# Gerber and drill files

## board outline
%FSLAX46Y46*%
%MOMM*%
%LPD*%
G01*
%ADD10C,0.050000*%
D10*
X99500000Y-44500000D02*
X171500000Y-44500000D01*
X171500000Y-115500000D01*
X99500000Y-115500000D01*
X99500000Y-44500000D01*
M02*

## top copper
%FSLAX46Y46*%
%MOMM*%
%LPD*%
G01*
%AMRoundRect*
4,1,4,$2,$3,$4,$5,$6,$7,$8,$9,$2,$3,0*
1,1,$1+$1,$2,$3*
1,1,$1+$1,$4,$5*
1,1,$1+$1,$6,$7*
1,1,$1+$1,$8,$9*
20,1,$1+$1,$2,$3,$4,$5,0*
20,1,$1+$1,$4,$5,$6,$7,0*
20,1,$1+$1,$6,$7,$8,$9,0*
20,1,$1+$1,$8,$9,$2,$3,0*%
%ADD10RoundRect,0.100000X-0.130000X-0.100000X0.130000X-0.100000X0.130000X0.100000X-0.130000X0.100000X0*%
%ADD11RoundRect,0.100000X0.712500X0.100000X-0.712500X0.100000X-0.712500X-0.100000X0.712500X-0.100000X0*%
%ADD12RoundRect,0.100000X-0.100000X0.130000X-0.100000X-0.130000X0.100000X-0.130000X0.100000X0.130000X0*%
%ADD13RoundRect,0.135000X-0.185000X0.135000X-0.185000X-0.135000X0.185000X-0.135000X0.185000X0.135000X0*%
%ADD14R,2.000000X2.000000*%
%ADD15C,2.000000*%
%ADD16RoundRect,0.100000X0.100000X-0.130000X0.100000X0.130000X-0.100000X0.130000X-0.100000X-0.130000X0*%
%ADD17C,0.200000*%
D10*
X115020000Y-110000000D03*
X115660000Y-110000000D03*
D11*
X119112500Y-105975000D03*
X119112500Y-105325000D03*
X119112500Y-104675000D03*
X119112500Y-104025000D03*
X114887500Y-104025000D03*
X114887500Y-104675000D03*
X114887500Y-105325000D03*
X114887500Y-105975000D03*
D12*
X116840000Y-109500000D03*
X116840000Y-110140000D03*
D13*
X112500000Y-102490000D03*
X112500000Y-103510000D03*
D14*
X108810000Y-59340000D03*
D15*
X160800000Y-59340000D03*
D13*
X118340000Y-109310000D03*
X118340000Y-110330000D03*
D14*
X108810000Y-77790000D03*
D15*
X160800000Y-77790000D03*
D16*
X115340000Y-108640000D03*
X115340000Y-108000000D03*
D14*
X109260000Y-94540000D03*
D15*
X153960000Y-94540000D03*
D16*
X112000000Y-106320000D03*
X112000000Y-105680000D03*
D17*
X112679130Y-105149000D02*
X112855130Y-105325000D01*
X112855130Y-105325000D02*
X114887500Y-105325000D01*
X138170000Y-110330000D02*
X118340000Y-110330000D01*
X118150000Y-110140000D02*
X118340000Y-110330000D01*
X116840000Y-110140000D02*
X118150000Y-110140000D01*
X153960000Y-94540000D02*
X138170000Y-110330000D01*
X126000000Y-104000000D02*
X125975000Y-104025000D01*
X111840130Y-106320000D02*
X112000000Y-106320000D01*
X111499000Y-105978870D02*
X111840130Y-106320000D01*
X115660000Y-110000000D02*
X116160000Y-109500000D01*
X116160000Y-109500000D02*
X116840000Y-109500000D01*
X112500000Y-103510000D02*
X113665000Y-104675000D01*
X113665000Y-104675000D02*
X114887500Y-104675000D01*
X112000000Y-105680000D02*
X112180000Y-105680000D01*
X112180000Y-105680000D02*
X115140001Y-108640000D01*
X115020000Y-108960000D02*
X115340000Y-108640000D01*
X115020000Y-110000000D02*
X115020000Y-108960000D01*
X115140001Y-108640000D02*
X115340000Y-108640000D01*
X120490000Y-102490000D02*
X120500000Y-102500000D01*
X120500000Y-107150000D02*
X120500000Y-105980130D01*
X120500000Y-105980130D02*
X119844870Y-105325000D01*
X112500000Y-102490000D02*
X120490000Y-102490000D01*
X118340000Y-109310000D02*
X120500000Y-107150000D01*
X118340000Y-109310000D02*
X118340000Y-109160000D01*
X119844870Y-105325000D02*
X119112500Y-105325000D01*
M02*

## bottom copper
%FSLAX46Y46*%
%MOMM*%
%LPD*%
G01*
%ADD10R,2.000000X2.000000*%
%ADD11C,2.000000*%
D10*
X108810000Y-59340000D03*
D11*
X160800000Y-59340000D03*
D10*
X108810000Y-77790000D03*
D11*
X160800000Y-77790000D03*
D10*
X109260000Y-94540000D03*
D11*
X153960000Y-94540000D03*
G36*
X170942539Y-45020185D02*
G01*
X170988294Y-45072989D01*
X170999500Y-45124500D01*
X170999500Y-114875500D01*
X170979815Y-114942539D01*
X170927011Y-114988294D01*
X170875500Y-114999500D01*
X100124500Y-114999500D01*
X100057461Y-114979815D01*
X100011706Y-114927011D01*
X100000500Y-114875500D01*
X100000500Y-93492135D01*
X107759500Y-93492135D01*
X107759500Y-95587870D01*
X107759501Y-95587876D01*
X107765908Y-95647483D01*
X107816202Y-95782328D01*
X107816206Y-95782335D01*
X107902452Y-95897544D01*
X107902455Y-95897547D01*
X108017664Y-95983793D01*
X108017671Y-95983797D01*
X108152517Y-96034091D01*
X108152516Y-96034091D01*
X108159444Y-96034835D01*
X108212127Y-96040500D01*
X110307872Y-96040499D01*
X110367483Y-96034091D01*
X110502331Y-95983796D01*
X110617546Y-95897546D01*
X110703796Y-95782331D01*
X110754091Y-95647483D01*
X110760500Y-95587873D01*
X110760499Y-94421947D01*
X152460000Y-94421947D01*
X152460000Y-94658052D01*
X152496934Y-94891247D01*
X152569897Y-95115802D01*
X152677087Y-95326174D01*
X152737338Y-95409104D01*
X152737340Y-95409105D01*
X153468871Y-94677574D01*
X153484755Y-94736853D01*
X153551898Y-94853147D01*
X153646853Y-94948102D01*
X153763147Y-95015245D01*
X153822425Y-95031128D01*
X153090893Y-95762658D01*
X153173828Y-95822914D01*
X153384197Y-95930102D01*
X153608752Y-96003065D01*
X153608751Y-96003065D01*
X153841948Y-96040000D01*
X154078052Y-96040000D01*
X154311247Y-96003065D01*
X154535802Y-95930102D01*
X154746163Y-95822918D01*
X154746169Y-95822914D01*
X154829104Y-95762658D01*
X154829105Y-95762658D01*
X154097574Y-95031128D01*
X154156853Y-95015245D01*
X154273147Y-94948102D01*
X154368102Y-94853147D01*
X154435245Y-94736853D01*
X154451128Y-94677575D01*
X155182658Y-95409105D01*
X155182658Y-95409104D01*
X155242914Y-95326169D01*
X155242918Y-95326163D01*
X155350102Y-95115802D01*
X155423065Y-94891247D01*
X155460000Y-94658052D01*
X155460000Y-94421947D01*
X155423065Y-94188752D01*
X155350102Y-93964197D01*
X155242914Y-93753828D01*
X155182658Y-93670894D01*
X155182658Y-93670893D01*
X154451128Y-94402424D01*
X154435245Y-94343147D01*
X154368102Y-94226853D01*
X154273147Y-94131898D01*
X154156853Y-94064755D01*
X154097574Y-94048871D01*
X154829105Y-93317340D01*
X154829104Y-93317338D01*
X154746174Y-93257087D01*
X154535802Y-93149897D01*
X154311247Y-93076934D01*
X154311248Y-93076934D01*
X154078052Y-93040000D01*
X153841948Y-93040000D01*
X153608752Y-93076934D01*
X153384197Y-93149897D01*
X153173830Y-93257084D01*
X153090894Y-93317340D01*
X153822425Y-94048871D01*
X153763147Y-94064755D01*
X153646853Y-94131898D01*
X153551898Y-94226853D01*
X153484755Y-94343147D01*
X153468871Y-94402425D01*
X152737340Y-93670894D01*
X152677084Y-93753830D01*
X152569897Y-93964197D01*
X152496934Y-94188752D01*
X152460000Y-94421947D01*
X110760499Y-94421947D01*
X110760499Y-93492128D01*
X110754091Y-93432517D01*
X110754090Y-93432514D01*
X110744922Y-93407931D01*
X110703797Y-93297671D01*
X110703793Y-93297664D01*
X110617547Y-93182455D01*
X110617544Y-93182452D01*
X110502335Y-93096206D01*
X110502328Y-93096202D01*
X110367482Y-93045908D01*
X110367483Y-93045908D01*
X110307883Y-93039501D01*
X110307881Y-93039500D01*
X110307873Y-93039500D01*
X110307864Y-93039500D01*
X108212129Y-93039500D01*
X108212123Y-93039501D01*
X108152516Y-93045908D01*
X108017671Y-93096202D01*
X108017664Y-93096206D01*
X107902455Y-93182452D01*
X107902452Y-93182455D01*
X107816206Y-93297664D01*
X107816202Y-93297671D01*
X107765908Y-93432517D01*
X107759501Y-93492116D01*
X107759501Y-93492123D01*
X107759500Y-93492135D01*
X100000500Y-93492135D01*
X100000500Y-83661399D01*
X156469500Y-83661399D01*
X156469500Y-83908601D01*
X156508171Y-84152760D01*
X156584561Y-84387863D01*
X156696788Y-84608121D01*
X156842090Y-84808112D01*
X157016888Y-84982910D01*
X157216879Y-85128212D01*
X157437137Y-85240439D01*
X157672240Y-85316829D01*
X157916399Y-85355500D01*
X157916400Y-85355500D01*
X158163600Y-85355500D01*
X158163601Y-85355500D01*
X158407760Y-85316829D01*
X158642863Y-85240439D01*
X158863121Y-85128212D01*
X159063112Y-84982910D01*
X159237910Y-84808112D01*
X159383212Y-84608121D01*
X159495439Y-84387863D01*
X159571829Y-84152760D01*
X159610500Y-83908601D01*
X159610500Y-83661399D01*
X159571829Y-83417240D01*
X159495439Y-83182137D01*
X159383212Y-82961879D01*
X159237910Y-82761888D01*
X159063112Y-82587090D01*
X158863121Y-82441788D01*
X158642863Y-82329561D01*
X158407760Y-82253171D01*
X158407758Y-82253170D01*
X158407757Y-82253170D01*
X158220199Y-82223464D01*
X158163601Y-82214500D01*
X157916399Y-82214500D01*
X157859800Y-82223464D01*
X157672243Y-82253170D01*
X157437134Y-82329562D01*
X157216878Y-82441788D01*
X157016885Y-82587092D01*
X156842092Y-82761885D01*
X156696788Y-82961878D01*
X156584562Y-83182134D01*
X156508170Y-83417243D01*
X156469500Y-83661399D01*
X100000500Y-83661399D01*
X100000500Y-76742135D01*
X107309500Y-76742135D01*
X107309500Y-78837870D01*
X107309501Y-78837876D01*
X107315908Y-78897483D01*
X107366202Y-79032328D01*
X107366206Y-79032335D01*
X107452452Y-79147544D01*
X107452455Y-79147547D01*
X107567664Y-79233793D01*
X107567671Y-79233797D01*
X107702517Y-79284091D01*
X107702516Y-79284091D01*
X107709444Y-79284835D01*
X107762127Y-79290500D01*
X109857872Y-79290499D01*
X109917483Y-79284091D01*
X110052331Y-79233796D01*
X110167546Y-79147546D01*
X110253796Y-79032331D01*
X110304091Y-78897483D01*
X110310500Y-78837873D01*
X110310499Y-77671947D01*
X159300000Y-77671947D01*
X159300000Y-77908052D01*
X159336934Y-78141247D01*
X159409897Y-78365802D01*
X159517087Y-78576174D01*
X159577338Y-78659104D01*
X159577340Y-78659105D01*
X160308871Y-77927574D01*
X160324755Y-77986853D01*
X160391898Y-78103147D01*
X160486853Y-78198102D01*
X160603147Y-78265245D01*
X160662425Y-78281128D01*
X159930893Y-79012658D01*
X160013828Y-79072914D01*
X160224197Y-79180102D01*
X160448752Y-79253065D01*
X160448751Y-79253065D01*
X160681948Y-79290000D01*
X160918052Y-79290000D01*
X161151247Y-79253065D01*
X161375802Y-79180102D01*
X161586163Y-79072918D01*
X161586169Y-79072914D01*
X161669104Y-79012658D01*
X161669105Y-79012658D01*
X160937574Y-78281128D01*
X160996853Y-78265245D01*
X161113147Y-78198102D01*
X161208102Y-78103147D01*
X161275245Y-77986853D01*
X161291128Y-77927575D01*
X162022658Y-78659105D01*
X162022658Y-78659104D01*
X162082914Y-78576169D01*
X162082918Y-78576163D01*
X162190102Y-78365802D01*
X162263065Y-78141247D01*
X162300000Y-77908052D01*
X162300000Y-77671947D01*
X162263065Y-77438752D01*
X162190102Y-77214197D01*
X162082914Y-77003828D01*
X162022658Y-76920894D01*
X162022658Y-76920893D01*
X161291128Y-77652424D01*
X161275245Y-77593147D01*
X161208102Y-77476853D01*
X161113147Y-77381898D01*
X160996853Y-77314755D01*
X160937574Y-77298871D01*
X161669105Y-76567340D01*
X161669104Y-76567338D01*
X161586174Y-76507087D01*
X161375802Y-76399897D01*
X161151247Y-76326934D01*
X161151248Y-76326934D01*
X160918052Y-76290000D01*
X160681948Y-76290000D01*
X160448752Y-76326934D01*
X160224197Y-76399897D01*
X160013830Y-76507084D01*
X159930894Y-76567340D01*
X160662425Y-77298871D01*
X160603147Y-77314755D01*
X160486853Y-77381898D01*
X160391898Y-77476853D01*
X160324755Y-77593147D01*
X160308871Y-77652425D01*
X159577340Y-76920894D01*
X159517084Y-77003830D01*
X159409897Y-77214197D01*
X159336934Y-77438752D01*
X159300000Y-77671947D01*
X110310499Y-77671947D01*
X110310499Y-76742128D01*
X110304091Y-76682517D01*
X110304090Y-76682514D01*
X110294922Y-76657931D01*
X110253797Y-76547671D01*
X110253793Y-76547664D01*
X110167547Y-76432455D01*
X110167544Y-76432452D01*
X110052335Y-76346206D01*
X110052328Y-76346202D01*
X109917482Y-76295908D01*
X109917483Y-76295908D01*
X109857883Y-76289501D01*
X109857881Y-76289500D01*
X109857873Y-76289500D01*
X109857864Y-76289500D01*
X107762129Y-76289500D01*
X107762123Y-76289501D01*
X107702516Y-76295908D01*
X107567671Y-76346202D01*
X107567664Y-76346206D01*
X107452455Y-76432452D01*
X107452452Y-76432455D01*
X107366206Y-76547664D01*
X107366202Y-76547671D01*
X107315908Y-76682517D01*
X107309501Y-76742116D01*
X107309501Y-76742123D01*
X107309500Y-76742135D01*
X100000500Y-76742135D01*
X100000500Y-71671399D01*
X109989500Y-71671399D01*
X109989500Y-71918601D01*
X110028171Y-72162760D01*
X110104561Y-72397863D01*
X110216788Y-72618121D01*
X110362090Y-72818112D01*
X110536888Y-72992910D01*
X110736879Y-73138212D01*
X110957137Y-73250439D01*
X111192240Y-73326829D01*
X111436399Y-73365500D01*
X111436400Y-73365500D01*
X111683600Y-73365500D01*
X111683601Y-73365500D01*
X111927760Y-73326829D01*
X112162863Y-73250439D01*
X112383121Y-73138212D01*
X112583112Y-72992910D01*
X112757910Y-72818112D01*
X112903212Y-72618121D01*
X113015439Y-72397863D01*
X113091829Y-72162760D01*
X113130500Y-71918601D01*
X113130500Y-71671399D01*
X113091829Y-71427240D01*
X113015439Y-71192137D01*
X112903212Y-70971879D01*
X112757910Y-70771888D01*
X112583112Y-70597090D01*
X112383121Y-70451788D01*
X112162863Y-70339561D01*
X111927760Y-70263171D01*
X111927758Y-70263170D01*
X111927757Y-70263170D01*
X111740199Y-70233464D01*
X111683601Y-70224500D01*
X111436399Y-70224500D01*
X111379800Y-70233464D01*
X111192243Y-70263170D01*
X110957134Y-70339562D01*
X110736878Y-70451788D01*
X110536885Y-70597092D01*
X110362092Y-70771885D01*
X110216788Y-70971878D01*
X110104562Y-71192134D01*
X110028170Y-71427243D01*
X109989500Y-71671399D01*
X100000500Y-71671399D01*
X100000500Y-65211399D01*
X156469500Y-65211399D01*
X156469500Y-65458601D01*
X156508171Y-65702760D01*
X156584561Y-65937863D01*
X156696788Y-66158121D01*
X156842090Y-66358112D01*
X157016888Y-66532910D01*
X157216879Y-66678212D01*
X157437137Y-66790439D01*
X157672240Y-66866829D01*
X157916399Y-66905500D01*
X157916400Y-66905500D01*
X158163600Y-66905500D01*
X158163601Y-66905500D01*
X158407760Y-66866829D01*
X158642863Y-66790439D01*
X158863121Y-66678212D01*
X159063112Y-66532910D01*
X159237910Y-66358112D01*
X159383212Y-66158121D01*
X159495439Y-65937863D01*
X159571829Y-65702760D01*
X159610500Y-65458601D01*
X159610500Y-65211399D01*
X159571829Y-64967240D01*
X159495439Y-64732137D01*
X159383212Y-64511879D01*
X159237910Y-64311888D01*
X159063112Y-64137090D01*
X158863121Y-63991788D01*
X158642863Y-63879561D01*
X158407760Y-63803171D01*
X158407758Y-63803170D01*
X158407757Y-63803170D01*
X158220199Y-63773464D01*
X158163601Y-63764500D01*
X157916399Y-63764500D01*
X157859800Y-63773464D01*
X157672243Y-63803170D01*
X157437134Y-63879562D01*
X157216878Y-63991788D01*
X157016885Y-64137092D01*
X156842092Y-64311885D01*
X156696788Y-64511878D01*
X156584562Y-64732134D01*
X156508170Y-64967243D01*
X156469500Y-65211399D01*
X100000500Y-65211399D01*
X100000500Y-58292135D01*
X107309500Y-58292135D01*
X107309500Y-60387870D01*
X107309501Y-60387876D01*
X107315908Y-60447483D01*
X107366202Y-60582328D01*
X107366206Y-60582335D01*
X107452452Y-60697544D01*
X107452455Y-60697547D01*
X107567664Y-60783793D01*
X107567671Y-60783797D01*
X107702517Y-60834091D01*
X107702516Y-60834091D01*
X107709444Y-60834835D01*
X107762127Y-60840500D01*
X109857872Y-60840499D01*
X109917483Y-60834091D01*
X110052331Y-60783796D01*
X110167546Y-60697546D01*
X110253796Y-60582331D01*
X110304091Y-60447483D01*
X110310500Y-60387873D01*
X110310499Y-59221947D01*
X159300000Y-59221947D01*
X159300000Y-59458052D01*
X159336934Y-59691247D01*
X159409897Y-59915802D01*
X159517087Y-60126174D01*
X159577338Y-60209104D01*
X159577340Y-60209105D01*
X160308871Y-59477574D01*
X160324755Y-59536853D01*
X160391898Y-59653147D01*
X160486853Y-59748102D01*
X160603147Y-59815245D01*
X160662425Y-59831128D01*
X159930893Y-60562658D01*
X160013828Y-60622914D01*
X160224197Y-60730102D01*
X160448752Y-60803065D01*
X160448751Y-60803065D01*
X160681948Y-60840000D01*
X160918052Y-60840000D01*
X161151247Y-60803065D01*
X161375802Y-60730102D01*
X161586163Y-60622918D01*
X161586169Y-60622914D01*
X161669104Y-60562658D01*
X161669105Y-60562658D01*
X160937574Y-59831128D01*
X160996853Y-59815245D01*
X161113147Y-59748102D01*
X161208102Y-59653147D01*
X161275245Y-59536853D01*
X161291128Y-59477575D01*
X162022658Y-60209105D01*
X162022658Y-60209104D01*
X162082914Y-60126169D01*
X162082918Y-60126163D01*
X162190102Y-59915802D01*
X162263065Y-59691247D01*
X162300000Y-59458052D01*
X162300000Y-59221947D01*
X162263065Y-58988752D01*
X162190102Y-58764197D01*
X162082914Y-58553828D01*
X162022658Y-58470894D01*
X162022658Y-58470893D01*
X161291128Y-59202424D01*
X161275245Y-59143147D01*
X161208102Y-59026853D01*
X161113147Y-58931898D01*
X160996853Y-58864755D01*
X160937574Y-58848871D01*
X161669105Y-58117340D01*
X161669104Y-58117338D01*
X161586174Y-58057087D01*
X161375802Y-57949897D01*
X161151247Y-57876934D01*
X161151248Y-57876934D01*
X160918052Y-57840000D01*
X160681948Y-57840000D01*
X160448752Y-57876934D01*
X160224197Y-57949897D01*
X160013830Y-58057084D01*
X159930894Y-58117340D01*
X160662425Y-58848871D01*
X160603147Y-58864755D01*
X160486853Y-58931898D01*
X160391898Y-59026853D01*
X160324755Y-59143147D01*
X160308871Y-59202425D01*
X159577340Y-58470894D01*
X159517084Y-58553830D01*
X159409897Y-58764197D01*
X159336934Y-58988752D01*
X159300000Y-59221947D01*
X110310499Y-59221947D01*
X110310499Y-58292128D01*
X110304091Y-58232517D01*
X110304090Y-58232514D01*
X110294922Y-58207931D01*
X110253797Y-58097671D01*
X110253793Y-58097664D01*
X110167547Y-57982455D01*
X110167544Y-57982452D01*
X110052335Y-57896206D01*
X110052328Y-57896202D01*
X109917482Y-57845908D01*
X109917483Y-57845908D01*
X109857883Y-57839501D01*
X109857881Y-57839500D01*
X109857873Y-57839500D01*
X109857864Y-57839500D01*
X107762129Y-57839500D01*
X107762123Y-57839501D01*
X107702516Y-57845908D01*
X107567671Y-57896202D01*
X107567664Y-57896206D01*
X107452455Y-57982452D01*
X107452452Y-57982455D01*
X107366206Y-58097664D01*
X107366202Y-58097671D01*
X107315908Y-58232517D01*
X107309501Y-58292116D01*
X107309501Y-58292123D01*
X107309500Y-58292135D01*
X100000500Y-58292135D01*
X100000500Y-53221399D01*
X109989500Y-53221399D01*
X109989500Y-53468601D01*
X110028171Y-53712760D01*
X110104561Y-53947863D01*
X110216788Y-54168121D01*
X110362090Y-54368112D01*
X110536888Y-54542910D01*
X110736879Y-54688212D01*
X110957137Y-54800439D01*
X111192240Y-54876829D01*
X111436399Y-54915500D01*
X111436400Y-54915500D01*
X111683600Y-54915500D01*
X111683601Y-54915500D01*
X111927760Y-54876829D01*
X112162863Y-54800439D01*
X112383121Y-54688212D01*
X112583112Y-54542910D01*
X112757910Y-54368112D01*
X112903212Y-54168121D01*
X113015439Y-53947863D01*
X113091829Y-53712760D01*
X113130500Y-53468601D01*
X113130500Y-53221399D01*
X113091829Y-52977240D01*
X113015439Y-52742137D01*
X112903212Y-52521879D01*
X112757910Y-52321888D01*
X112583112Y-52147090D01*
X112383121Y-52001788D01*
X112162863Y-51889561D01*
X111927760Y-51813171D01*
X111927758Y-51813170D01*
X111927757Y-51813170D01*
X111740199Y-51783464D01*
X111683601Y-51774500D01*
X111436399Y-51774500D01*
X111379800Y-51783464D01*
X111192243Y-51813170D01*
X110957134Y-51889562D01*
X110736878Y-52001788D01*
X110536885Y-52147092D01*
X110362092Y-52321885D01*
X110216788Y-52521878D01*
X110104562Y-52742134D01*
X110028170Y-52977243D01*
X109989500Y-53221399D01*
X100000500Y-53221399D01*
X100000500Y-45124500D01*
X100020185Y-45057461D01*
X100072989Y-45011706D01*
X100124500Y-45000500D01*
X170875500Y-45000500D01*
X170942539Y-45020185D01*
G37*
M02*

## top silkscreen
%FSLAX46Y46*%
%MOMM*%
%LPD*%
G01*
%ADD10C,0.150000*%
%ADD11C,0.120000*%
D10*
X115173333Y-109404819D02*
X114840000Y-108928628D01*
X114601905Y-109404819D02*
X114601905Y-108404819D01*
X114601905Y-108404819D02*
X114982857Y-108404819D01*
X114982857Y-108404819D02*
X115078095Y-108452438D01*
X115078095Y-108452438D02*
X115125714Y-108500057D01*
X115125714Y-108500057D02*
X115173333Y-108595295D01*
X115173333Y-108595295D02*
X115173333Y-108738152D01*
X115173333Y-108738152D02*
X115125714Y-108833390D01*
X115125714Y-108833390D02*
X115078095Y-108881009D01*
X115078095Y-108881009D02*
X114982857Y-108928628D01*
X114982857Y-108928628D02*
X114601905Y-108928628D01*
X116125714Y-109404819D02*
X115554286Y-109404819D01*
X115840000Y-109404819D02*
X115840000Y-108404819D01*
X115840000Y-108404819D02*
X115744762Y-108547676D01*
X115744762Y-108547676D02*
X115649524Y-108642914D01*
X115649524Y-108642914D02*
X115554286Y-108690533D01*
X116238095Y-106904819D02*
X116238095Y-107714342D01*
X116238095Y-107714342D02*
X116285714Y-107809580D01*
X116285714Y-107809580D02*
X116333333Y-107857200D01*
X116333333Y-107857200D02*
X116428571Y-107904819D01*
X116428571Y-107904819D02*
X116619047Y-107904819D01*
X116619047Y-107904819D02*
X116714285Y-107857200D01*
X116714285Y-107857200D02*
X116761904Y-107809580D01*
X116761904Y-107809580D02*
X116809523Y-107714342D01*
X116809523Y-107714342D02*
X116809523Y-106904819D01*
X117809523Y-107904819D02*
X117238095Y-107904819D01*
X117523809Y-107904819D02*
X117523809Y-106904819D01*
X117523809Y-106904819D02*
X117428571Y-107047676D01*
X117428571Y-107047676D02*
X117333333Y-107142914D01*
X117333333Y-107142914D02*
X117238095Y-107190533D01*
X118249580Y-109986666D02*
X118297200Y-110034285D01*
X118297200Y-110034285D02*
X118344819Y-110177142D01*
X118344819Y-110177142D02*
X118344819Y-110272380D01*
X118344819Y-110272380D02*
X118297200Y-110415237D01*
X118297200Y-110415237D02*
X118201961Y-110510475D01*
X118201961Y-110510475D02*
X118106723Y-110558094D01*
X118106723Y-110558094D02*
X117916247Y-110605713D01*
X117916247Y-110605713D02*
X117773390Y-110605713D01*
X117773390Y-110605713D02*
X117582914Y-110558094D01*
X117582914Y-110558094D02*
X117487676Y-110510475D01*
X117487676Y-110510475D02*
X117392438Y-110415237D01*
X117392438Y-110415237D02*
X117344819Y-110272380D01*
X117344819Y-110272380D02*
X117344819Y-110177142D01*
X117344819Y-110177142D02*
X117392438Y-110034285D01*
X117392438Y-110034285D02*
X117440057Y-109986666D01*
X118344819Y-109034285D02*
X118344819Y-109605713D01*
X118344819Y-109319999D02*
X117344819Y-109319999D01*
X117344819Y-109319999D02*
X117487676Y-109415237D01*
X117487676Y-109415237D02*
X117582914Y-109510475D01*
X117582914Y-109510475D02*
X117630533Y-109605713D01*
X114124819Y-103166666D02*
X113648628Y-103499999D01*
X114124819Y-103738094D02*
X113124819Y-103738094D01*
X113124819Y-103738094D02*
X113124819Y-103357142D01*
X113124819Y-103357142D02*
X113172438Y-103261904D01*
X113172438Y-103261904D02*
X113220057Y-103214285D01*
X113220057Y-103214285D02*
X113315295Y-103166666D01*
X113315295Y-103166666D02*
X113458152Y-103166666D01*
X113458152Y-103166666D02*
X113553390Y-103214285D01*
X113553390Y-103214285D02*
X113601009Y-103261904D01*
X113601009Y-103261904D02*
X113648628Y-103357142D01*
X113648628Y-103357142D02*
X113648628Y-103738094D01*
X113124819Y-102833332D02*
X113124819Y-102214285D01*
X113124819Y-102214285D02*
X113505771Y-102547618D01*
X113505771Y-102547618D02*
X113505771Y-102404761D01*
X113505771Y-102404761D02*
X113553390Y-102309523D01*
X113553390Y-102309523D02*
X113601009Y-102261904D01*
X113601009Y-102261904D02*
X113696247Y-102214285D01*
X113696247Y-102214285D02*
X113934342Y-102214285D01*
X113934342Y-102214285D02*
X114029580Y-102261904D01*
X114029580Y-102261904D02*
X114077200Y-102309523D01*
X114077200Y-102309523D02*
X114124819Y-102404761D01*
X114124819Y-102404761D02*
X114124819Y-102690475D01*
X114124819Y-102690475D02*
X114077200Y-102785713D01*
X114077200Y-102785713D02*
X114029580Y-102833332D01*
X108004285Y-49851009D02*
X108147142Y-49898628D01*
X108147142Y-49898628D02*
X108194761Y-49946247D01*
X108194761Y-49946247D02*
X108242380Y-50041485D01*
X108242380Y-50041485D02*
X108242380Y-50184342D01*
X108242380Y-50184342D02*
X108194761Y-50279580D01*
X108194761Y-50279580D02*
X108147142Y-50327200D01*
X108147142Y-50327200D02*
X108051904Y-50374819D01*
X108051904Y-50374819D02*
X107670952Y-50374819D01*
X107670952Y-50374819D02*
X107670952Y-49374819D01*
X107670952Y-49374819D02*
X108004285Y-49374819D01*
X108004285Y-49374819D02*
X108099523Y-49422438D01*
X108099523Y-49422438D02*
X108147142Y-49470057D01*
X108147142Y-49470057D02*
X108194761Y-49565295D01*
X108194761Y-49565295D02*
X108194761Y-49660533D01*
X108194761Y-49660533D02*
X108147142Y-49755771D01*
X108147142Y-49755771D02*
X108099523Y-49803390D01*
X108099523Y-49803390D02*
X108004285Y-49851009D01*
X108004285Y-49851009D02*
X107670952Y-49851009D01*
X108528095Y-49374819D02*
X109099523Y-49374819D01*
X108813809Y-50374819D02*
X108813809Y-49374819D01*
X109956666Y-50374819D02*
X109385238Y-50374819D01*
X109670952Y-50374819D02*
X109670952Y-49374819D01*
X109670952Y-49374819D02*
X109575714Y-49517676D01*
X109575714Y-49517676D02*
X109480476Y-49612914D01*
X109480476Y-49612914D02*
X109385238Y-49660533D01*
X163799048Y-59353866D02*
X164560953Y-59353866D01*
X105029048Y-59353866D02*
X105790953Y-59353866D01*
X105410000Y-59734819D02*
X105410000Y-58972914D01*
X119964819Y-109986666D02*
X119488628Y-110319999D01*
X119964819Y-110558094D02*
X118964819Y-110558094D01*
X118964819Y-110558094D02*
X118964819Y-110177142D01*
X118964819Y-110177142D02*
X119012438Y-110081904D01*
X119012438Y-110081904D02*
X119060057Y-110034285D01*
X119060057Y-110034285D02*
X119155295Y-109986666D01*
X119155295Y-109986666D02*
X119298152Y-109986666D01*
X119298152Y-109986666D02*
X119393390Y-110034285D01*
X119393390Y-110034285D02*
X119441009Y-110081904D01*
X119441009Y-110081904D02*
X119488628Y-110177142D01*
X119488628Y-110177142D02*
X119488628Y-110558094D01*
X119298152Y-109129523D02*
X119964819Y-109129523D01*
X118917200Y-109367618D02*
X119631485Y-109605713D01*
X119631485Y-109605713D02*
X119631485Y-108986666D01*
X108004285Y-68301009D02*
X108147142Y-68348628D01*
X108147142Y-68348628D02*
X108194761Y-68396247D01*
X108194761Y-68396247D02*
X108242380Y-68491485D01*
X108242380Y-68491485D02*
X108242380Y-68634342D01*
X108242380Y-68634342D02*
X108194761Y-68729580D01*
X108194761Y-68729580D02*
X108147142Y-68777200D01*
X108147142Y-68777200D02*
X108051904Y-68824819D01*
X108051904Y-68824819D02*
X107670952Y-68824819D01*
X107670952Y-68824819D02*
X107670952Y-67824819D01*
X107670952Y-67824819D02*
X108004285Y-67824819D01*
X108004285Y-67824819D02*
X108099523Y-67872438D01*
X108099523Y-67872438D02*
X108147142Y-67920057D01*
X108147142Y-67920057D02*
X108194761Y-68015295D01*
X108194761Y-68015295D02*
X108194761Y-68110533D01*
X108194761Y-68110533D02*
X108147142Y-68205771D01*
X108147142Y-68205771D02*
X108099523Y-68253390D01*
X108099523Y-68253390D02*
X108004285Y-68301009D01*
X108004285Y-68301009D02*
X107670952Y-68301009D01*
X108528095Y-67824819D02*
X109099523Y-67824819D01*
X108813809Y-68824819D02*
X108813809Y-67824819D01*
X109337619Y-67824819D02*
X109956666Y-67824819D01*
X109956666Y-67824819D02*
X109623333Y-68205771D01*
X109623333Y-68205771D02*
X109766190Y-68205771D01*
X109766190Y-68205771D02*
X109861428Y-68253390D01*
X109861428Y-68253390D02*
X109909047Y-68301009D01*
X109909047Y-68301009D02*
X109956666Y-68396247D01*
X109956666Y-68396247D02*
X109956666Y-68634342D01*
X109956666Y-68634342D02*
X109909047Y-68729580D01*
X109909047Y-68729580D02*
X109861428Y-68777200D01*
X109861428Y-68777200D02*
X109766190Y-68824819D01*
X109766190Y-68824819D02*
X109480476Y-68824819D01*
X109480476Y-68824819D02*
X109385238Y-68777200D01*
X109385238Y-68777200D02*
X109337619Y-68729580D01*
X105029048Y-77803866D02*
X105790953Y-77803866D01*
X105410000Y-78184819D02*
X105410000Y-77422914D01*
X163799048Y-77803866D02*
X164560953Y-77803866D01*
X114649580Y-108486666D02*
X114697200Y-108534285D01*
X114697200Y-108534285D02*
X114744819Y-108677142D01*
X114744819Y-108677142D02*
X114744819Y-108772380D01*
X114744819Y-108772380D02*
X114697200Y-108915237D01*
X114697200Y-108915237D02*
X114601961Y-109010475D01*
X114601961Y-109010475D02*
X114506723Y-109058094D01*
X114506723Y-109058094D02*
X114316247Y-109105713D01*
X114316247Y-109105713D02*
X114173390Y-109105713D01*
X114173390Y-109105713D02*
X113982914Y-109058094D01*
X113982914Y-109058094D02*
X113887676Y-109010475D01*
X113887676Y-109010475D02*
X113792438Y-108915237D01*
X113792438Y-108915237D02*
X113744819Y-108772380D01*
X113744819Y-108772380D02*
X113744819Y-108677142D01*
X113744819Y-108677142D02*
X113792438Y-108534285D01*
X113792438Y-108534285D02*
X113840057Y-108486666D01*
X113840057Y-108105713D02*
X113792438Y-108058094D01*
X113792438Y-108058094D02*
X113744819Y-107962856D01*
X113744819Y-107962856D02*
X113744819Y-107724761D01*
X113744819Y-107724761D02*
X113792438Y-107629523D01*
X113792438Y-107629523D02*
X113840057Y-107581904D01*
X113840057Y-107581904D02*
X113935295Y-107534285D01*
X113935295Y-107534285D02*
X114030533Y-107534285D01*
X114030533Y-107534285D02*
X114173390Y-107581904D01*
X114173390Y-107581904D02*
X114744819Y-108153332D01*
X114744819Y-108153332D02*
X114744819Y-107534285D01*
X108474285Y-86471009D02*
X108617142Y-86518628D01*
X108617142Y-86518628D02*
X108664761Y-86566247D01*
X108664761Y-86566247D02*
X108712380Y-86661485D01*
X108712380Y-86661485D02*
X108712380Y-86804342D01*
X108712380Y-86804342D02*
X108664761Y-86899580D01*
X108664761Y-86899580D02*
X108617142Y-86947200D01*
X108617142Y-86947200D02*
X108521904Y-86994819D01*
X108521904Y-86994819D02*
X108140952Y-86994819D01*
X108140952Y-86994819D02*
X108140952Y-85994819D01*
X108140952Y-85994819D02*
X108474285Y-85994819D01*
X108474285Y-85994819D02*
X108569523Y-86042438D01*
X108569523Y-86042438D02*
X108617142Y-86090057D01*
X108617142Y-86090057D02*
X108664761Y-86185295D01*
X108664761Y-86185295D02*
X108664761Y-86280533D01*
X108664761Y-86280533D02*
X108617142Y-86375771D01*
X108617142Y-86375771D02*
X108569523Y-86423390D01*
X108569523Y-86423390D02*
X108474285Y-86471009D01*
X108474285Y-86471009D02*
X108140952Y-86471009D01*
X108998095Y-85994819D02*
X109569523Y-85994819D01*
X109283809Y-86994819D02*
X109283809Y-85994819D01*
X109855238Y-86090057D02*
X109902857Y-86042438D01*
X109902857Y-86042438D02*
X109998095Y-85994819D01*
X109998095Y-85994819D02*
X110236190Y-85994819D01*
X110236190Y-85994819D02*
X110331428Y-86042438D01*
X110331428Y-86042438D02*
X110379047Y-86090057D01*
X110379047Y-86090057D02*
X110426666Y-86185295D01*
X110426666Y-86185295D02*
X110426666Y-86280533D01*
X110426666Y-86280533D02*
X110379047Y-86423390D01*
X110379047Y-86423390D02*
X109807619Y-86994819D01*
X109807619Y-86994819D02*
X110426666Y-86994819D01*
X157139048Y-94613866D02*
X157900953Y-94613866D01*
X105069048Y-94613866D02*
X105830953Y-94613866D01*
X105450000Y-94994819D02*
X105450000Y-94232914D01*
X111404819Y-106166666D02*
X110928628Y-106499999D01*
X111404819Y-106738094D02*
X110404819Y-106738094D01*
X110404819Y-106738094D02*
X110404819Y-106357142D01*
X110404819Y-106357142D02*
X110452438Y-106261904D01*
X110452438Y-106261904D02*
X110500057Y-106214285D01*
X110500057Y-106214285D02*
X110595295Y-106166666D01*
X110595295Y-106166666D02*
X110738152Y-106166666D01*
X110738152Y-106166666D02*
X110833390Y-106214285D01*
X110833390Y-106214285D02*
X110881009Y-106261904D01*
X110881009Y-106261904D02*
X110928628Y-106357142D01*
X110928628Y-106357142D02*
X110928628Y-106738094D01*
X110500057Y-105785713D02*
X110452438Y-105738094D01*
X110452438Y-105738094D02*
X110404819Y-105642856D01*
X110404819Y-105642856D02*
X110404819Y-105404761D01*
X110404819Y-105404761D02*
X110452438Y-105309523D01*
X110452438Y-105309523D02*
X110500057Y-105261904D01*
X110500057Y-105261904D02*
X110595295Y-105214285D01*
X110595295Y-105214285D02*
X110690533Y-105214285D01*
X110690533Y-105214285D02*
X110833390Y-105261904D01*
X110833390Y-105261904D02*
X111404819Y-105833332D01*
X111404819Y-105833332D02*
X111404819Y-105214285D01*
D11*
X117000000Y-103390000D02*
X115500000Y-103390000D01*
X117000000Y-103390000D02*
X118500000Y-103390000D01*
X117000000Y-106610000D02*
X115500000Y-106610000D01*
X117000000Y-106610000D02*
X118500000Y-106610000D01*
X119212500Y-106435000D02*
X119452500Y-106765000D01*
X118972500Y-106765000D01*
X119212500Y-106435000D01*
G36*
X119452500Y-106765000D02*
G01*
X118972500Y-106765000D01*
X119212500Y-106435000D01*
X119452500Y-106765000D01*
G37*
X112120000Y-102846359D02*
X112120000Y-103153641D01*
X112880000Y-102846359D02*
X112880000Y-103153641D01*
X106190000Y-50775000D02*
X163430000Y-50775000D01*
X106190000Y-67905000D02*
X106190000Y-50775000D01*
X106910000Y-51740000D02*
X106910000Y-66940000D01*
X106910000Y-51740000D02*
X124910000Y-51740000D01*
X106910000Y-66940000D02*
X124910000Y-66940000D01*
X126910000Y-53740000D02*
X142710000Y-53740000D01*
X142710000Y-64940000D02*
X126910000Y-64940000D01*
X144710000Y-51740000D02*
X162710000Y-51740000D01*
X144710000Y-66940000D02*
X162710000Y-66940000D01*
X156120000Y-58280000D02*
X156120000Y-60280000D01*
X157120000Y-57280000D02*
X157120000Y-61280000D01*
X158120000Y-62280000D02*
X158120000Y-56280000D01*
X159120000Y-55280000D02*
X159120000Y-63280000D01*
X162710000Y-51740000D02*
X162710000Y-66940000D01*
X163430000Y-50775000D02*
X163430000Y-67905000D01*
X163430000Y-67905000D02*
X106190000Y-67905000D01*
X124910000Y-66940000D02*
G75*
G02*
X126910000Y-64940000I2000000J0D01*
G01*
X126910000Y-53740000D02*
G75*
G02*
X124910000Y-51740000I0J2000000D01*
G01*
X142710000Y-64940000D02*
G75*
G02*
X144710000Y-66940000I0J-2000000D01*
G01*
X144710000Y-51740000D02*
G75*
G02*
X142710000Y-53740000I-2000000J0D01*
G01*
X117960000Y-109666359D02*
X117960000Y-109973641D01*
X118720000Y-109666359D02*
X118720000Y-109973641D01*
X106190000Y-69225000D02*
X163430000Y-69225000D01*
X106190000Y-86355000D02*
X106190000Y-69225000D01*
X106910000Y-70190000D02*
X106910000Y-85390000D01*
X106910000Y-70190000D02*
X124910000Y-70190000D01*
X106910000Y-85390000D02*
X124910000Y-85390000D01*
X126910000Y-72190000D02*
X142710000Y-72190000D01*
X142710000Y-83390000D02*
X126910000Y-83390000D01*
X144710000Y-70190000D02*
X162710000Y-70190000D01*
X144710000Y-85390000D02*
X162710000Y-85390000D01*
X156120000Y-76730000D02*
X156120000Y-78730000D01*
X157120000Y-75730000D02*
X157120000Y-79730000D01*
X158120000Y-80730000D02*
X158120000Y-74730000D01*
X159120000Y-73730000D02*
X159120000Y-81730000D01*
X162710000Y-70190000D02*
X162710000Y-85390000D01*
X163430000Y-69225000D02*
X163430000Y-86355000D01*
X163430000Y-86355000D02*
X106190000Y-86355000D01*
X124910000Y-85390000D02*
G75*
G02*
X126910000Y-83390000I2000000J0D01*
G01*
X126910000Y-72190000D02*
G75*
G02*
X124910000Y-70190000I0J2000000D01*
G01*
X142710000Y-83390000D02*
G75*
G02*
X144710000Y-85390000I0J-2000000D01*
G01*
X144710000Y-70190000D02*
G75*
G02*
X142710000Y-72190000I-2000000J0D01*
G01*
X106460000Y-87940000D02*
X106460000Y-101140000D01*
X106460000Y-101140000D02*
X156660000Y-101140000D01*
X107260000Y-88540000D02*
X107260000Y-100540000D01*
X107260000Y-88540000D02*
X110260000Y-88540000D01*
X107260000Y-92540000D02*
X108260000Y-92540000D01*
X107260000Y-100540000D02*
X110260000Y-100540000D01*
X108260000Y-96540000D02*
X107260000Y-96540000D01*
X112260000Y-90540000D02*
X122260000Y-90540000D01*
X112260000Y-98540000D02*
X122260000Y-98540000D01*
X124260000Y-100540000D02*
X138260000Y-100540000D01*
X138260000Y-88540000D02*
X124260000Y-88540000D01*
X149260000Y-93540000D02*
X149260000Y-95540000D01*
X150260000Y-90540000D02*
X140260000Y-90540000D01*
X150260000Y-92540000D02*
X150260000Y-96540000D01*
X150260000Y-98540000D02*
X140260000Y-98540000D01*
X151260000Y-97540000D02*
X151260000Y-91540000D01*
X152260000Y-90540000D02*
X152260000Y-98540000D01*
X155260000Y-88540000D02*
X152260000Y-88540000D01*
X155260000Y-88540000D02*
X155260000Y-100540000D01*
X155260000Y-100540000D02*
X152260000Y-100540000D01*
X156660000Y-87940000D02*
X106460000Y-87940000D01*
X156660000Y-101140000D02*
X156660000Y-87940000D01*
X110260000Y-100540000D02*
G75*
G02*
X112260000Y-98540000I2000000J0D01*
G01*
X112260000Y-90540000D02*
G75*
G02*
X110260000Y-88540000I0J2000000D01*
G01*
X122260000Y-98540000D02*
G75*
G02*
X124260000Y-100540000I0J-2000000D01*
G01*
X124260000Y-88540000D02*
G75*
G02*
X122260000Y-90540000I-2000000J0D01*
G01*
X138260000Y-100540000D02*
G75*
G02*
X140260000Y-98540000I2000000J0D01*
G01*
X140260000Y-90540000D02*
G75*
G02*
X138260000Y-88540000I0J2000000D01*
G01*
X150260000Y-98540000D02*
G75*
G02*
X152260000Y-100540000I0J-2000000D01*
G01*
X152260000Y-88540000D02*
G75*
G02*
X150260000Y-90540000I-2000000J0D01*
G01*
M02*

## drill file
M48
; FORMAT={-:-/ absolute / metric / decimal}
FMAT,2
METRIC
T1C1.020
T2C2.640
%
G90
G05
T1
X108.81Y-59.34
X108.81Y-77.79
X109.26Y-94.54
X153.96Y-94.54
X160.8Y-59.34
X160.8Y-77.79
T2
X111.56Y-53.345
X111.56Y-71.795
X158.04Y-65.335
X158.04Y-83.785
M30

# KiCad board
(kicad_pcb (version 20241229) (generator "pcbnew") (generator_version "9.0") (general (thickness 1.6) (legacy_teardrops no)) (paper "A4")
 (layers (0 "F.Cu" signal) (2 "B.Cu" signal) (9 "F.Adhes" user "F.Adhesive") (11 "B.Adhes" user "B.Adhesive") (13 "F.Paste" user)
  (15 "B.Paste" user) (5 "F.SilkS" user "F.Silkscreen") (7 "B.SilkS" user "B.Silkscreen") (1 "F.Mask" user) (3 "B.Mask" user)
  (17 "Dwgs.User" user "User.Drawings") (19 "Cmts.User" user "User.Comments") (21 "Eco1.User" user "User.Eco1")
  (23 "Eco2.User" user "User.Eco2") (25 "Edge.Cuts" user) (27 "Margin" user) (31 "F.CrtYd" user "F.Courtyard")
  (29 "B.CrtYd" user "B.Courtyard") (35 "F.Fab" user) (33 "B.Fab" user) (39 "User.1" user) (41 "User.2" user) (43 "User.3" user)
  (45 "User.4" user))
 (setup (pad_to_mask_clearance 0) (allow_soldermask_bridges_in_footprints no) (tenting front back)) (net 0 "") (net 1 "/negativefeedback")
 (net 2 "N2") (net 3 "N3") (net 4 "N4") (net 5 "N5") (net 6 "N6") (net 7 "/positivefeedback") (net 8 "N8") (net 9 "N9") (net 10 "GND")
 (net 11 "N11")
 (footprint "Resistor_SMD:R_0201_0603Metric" (layer "F.Cu") (at 115.34 110)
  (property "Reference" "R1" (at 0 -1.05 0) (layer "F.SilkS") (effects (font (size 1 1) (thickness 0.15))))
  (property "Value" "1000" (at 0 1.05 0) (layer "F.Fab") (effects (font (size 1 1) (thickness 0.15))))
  (pad "" smd roundrect (at -0.345 0) (size 0.318 0.36) (layers "F.Paste") (roundrect_rratio 0.25))
  (pad "" smd roundrect (at 0.345 0) (size 0.318 0.36) (layers "F.Paste") (roundrect_rratio 0.25))
  (pad "1" smd roundrect (at -0.32 0) (size 0.46 0.4) (layers "F.Cu" "F.Mask") (roundrect_rratio 0.25) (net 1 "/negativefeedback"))
  (pad "2" smd roundrect (at 0.32 0) (size 0.46 0.4) (layers "F.Cu" "F.Mask") (roundrect_rratio 0.25) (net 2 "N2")))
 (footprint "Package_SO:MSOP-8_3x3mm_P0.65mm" (layer "F.Cu") (at 117 105 180)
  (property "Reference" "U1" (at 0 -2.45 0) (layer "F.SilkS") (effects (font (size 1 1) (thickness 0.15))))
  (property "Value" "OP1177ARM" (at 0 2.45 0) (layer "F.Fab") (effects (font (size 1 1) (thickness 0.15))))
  (fp_line (start 0 1.61) (end 1.5 1.61) (stroke (width 0.12) (type solid)) (layer "F.SilkS"))
  (fp_line (start 0 1.61) (end -1.5 1.61) (stroke (width 0.12) (type solid)) (layer "F.SilkS"))
  (fp_line (start 0 -1.61) (end 1.5 -1.61) (stroke (width 0.12) (type solid)) (layer "F.SilkS"))
  (fp_line (start 0 -1.61) (end -1.5 -1.61) (stroke (width 0.12) (type solid)) (layer "F.SilkS"))
  (fp_poly
   (pts (xy -2.2125 -1.435) (xy -2.4525 -1.765) (xy -1.9725 -1.765)) (stroke (width 0.12) (type solid)) (fill yes) (layer "F.SilkS"))
  (pad "1" smd roundrect (at -2.1125 -0.975 180) (size 1.625 0.4) (layers "F.Cu" "F.Mask" "F.Paste") (roundrect_rratio 0.25) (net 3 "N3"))
  (pad "2" smd roundrect (at -2.1125 -0.325 180) (size 1.625 0.4) (layers "F.Cu" "F.Mask" "F.Paste") (roundrect_rratio 0.25) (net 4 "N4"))
  (pad "3" smd roundrect (at -2.1125 0.325 180) (size 1.625 0.4) (layers "F.Cu" "F.Mask" "F.Paste") (roundrect_rratio 0.25) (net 2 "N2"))
  (pad "4" smd roundrect (at -2.1125 0.975 180) (size 1.625 0.4) (layers "F.Cu" "F.Mask" "F.Paste") (roundrect_rratio 0.25) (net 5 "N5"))
  (pad "5" smd roundrect (at 2.1125 0.975 180) (size 1.625 0.4) (layers "F.Cu" "F.Mask" "F.Paste") (roundrect_rratio 0.25) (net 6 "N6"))
  (pad "6" smd roundrect (at 2.1125 0.325 180) (size 1.625 0.4) (layers "F.Cu" "F.Mask" "F.Paste") (roundrect_rratio 0.25)
   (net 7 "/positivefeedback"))
  (pad "7" smd roundrect (at 2.1125 -0.325 180) (size 1.625 0.4) (layers "F.Cu" "F.Mask" "F.Paste") (roundrect_rratio 0.25) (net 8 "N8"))
  (pad "8" smd roundrect (at 2.1125 -0.975 180) (size 1.625 0.4) (layers "F.Cu" "F.Mask" "F.Paste") (roundrect_rratio 0.25) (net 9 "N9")))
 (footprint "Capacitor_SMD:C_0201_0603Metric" (layer "F.Cu") (at 116.84 109.82 -90)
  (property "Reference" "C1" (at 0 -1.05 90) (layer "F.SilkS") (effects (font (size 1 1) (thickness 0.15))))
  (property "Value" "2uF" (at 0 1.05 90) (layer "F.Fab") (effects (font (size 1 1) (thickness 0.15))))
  (pad "" smd roundrect (at -0.345 0 270) (size 0.318 0.36) (layers "F.Paste") (roundrect_rratio 0.25))
  (pad "" smd roundrect (at 0.345 0 270) (size 0.318 0.36) (layers "F.Paste") (roundrect_rratio 0.25))
  (pad "1" smd roundrect (at -0.32 0 270) (size 0.46 0.4) (layers "F.Cu" "F.Mask") (roundrect_rratio 0.25) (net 2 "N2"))
  (pad "2" smd roundrect (at 0.32 0 270) (size 0.46 0.4) (layers "F.Cu" "F.Mask") (roundrect_rratio 0.25) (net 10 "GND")))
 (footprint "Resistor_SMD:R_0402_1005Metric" (layer "F.Cu") (at 112.5 103 -90)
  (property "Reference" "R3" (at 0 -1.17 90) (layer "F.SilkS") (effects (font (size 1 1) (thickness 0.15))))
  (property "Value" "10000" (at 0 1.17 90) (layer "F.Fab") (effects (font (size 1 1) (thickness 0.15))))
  (fp_line (start -0.153641 0.38) (end 0.153641 0.38) (stroke (width 0.12) (type solid)) (layer "F.SilkS"))
  (fp_line (start -0.153641 -0.38) (end 0.153641 -0.38) (stroke (width 0.12) (type solid)) (layer "F.SilkS"))
  (pad "1" smd roundrect (at -0.51 0 270) (size 0.54 0.64) (layers "F.Cu" "F.Mask" "F.Paste") (roundrect_rratio 0.25) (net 4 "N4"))
  (pad "2" smd roundrect (at 0.51 0 270) (size 0.54 0.64) (layers "F.Cu" "F.Mask" "F.Paste") (roundrect_rratio 0.25)
   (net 7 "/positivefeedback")))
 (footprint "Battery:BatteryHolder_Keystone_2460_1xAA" (layer "F.Cu") (at 108.81 59.34)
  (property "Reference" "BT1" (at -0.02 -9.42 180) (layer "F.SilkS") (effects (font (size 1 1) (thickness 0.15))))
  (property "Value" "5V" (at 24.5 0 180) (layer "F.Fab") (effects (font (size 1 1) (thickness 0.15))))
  (fp_line (start -2.62 -8.565) (end 54.62 -8.565) (stroke (width 0.12) (type solid)) (layer "F.SilkS"))
  (fp_line (start -2.62 8.565) (end -2.62 -8.565) (stroke (width 0.12) (type solid)) (layer "F.SilkS"))
  (fp_line (start -1.9 -7.6) (end -1.9 7.6) (stroke (width 0.12) (type solid)) (layer "F.SilkS"))
  (fp_line (start -1.9 -7.6) (end 16.1 -7.6) (stroke (width 0.12) (type solid)) (layer "F.SilkS"))
  (fp_line (start -1.9 7.6) (end 16.1 7.6) (stroke (width 0.12) (type solid)) (layer "F.SilkS"))
  (fp_line (start 18.1 -5.6) (end 33.9 -5.6) (stroke (width 0.12) (type solid)) (layer "F.SilkS"))
  (fp_line (start 33.9 5.6) (end 18.1 5.6) (stroke (width 0.12) (type solid)) (layer "F.SilkS"))
  (fp_line (start 35.9 -7.6) (end 53.9 -7.6) (stroke (width 0.12) (type solid)) (layer "F.SilkS"))
  (fp_line (start 35.9 7.6) (end 53.9 7.6) (stroke (width 0.12) (type solid)) (layer "F.SilkS"))
  (fp_line (start 47.31 -1.06) (end 47.31 0.94) (stroke (width 0.12) (type solid)) (layer "F.SilkS"))
  (fp_line (start 48.31 -2.06) (end 48.31 1.94) (stroke (width 0.12) (type solid)) (layer "F.SilkS"))
  (fp_line (start 49.31 2.94) (end 49.31 -3.06) (stroke (width 0.12) (type solid)) (layer "F.SilkS"))
  (fp_line (start 50.31 -4.06) (end 50.31 3.94) (stroke (width 0.12) (type solid)) (layer "F.SilkS"))
  (fp_line (start 53.9 -7.6) (end 53.9 7.6) (stroke (width 0.12) (type solid)) (layer "F.SilkS"))
  (fp_line (start 54.62 -8.565) (end 54.62 8.565) (stroke (width 0.12) (type solid)) (layer "F.SilkS"))
  (fp_line (start 54.62 8.565) (end -2.62 8.565) (stroke (width 0.12) (type solid)) (layer "F.SilkS"))
  (fp_arc (start 16.1 7.6) (mid 16.685786 6.185786) (end 18.1 5.6) (stroke (width 0.12) (type solid)) (layer "F.SilkS"))
  (fp_arc (start 18.1 -5.6) (mid 16.685786 -6.185786) (end 16.1 -7.6) (stroke (width 0.12) (type solid)) (layer "F.SilkS"))
  (fp_arc (start 33.9 5.6) (mid 35.314214 6.185786) (end 35.9 7.6) (stroke (width 0.12) (type solid)) (layer "F.SilkS"))
  (fp_arc (start 35.9 -7.6) (mid 35.314214 -6.185786) (end 33.9 -5.6) (stroke (width 0.12) (type solid)) (layer "F.SilkS"))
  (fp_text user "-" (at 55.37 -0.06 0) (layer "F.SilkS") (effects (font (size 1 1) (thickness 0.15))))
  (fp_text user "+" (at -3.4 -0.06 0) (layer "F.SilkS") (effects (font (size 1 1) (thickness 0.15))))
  (pad "" np_thru_hole circle (at 2.75 -5.995 90) (size 2.64 2.64) (drill 2.64) (layers "*.Cu" "*.Mask"))
  (pad "" np_thru_hole circle (at 49.23 5.995) (size 2.64 2.64) (drill 2.64) (layers "*.Cu" "*.Mask"))
  (pad "1" thru_hole rect (at 0 0 180) (size 2 2) (drill 1.02) (layers "*.Cu" "*.Mask") (remove_unused_layers no) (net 8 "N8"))
  (pad "2" thru_hole circle (at 51.99 0 180) (size 2 2) (drill 1.02) (layers "*.Cu" "*.Mask") (remove_unused_layers no) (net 10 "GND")))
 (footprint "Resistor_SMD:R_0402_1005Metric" (layer "F.Cu") (at 118.34 109.82 -90)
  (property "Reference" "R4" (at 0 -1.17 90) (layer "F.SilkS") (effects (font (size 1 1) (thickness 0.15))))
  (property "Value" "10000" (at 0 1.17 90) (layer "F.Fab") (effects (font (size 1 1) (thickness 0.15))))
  (fp_line (start -0.153641 0.38) (end 0.153641 0.38) (stroke (width 0.12) (type solid)) (layer "F.SilkS"))
  (fp_line (start -0.153641 -0.38) (end 0.153641 -0.38) (stroke (width 0.12) (type solid)) (layer "F.SilkS"))
  (pad "1" smd roundrect (at -0.51 0 270) (size 0.54 0.64) (layers "F.Cu" "F.Mask" "F.Paste") (roundrect_rratio 0.25) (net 4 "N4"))
  (pad "2" smd roundrect (at 0.51 0 270) (size 0.54 0.64) (layers "F.Cu" "F.Mask" "F.Paste") (roundrect_rratio 0.25) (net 10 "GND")))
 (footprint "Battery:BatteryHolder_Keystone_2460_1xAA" (layer "F.Cu") (at 108.81 77.79)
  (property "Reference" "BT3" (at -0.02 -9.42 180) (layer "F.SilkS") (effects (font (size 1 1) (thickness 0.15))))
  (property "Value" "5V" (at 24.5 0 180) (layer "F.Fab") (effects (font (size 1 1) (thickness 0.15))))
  (fp_line (start -2.62 -8.565) (end 54.62 -8.565) (stroke (width 0.12) (type solid)) (layer "F.SilkS"))
  (fp_line (start -2.62 8.565) (end -2.62 -8.565) (stroke (width 0.12) (type solid)) (layer "F.SilkS"))
  (fp_line (start -1.9 -7.6) (end -1.9 7.6) (stroke (width 0.12) (type solid)) (layer "F.SilkS"))
  (fp_line (start -1.9 -7.6) (end 16.1 -7.6) (stroke (width 0.12) (type solid)) (layer "F.SilkS"))
  (fp_line (start -1.9 7.6) (end 16.1 7.6) (stroke (width 0.12) (type solid)) (layer "F.SilkS"))
  (fp_line (start 18.1 -5.6) (end 33.9 -5.6) (stroke (width 0.12) (type solid)) (layer "F.SilkS"))
  (fp_line (start 33.9 5.6) (end 18.1 5.6) (stroke (width 0.12) (type solid)) (layer "F.SilkS"))
  (fp_line (start 35.9 -7.6) (end 53.9 -7.6) (stroke (width 0.12) (type solid)) (layer "F.SilkS"))
  (fp_line (start 35.9 7.6) (end 53.9 7.6) (stroke (width 0.12) (type solid)) (layer "F.SilkS"))
  (fp_line (start 47.31 -1.06) (end 47.31 0.94) (stroke (width 0.12) (type solid)) (layer "F.SilkS"))
  (fp_line (start 48.31 -2.06) (end 48.31 1.94) (stroke (width 0.12) (type solid)) (layer "F.SilkS"))
  (fp_line (start 49.31 2.94) (end 49.31 -3.06) (stroke (width 0.12) (type solid)) (layer "F.SilkS"))
  (fp_line (start 50.31 -4.06) (end 50.31 3.94) (stroke (width 0.12) (type solid)) (layer "F.SilkS"))
  (fp_line (start 53.9 -7.6) (end 53.9 7.6) (stroke (width 0.12) (type solid)) (layer "F.SilkS"))
  (fp_line (start 54.62 -8.565) (end 54.62 8.565) (stroke (width 0.12) (type solid)) (layer "F.SilkS"))
  (fp_line (start 54.62 8.565) (end -2.62 8.565) (stroke (width 0.12) (type solid)) (layer "F.SilkS"))
  (fp_arc (start 16.1 7.6) (mid 16.685786 6.185786) (end 18.1 5.6) (stroke (width 0.12) (type solid)) (layer "F.SilkS"))
  (fp_arc (start 18.1 -5.6) (mid 16.685786 -6.185786) (end 16.1 -7.6) (stroke (width 0.12) (type solid)) (layer "F.SilkS"))
  (fp_arc (start 33.9 5.6) (mid 35.314214 6.185786) (end 35.9 7.6) (stroke (width 0.12) (type solid)) (layer "F.SilkS"))
  (fp_arc (start 35.9 -7.6) (mid 35.314214 -6.185786) (end 33.9 -5.6) (stroke (width 0.12) (type solid)) (layer "F.SilkS"))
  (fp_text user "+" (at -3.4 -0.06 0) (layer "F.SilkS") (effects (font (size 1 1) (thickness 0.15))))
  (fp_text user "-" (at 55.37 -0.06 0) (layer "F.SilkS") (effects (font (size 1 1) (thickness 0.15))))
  (pad "" np_thru_hole circle (at 2.75 -5.995 90) (size 2.64 2.64) (drill 2.64) (layers "*.Cu" "*.Mask"))
  (pad "" np_thru_hole circle (at 49.23 5.995) (size 2.64 2.64) (drill 2.64) (layers "*.Cu" "*.Mask"))
  (pad "1" thru_hole rect (at 0 0 180) (size 2 2) (drill 1.02) (layers "*.Cu" "*.Mask") (remove_unused_layers no) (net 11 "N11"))
  (pad "2" thru_hole circle (at 51.99 0 180) (size 2 2) (drill 1.02) (layers "*.Cu" "*.Mask") (remove_unused_layers no) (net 10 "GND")))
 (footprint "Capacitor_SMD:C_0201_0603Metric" (layer "F.Cu") (at 115.34 108.32 90)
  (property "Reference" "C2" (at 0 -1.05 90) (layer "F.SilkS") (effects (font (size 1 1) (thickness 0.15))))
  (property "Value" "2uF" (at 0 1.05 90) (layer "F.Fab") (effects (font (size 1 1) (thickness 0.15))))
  (pad "" smd roundrect (at -0.345 0 90) (size 0.318 0.36) (layers "F.Paste") (roundrect_rratio 0.25))
  (pad "" smd roundrect (at 0.345 0 90) (size 0.318 0.36) (layers "F.Paste") (roundrect_rratio 0.25))
  (pad "1" smd roundrect (at -0.32 0 90) (size 0.46 0.4) (layers "F.Cu" "F.Mask") (roundrect_rratio 0.25) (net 1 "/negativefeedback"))
  (pad "2" smd roundrect (at 0.32 0 90) (size 0.46 0.4) (layers "F.Cu" "F.Mask") (roundrect_rratio 0.25) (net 7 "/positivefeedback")))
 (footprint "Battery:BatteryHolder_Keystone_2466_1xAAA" (layer "F.Cu") (at 109.26 94.54)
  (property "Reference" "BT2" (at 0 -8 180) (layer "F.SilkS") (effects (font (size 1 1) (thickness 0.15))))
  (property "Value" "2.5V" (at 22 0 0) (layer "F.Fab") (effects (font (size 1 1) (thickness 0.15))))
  (fp_line (start -2.8 -6.6) (end -2.8 6.6) (stroke (width 0.12) (type solid)) (layer "F.SilkS"))
  (fp_line (start -2.8 6.6) (end 47.4 6.6) (stroke (width 0.12) (type solid)) (layer "F.SilkS"))
  (fp_line (start -2 -6) (end -2 6) (stroke (width 0.12) (type solid)) (layer "F.SilkS"))
  (fp_line (start -2 -6) (end 1 -6) (stroke (width 0.12) (type solid)) (layer "F.SilkS"))
  (fp_line (start -2 -2) (end -1 -2) (stroke (width 0.12) (type solid)) (layer "F.SilkS"))
  (fp_line (start -2 6) (end 1 6) (stroke (width 0.12) (type solid)) (layer "F.SilkS"))
  (fp_line (start -1 2) (end -2 2) (stroke (width 0.12) (type solid)) (layer "F.SilkS"))
  (fp_line (start 3 -4) (end 13 -4) (stroke (width 0.12) (type solid)) (layer "F.SilkS"))
  (fp_line (start 3 4) (end 13 4) (stroke (width 0.12) (type solid)) (layer "F.SilkS"))
  (fp_line (start 15 6) (end 29 6) (stroke (width 0.12) (type solid)) (layer "F.SilkS"))
  (fp_line (start 29 -6) (end 15 -6) (stroke (width 0.12) (type solid)) (layer "F.SilkS"))
  (fp_line (start 40 -1) (end 40 1) (stroke (width 0.12) (type solid)) (layer "F.SilkS"))
  (fp_line (start 41 -4) (end 31 -4) (stroke (width 0.12) (type solid)) (layer "F.SilkS"))
  (fp_line (start 41 -2) (end 41 2) (stroke (width 0.12) (type solid)) (layer "F.SilkS"))
  (fp_line (start 41 4) (end 31 4) (stroke (width 0.12) (type solid)) (layer "F.SilkS"))
  (fp_line (start 42 3) (end 42 -3) (stroke (width 0.12) (type solid)) (layer "F.SilkS"))
  (fp_line (start 43 -4) (end 43 4) (stroke (width 0.12) (type solid)) (layer "F.SilkS"))
  (fp_line (start 46 -6) (end 43 -6) (stroke (width 0.12) (type solid)) (layer "F.SilkS"))
  (fp_line (start 46 -6) (end 46 6) (stroke (width 0.12) (type solid)) (layer "F.SilkS"))
  (fp_line (start 46 6) (end 43 6) (stroke (width 0.12) (type solid)) (layer "F.SilkS"))
  (fp_line (start 47.4 -6.6) (end -2.8 -6.6) (stroke (width 0.12) (type solid)) (layer "F.SilkS"))
  (fp_line (start 47.4 6.6) (end 47.4 -6.6) (stroke (width 0.12) (type solid)) (layer "F.SilkS"))
  (fp_arc (start 1 6) (mid 1.585786 4.585786) (end 3 4) (stroke (width 0.12) (type solid)) (layer "F.SilkS"))
  (fp_arc (start 3 -4) (mid 1.585786 -4.585786) (end 1 -6) (stroke (width 0.12) (type solid)) (layer "F.SilkS"))
  (fp_arc (start 13 4) (mid 14.414214 4.585786) (end 15 6) (stroke (width 0.12) (type solid)) (layer "F.SilkS"))
  (fp_arc (start 15 -6) (mid 14.414214 -4.585786) (end 13 -4) (stroke (width 0.12) (type solid)) (layer "F.SilkS"))
  (fp_arc (start 29 6) (mid 29.585786 4.585786) (end 31 4) (stroke (width 0.12) (type solid)) (layer "F.SilkS"))
  (fp_arc (start 31 -4) (mid 29.585786 -4.585786) (end 29 -6) (stroke (width 0.12) (type solid)) (layer "F.SilkS"))
  (fp_arc (start 41 4) (mid 42.414214 4.585786) (end 43 6) (stroke (width 0.12) (type solid)) (layer "F.SilkS"))
  (fp_arc (start 43 -6) (mid 42.414214 -4.585786) (end 41 -4) (stroke (width 0.12) (type solid)) (layer "F.SilkS"))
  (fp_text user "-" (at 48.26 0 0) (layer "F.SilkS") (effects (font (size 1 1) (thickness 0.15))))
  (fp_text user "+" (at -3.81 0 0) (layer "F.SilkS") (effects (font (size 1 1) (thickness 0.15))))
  (pad "1" thru_hole rect (at 0 0) (size 2 2) (drill 1.02) (layers "*.Cu" "*.Mask") (remove_unused_layers no) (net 5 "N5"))
  (pad "2" thru_hole circle (at 44.7 0) (size 2 2) (drill 1.02) (layers "*.Cu" "*.Mask") (remove_unused_layers no) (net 10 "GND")))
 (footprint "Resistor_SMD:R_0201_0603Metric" (layer "F.Cu") (at 112 106 90)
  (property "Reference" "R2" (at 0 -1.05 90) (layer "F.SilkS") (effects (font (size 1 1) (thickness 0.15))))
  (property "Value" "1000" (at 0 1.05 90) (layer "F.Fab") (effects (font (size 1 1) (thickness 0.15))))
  (pad "" smd roundrect (at -0.345 0 90) (size 0.318 0.36) (layers "F.Paste") (roundrect_rratio 0.25))
  (pad "" smd roundrect (at 0.345 0 90) (size 0.318 0.36) (layers "F.Paste") (roundrect_rratio 0.25))
  (pad "1" smd roundrect (at -0.32 0 90) (size 0.46 0.4) (layers "F.Cu" "F.Mask") (roundrect_rratio 0.25) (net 11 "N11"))
  (pad "2" smd roundrect (at 0.32 0 90) (size 0.46 0.4) (layers "F.Cu" "F.Mask") (roundrect_rratio 0.25) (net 1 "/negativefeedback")))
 (gr_rect (start 99.5 44.5) (end 171.5 115.5) (stroke (width 0.05) (type default)) (fill no) (layer "Edge.Cuts"))
 (segment (start 112.67913 105.149) (end 112.85513 105.325) (width 0.2) (layer "F.Cu") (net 8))
 (segment (start 112.85513 105.325) (end 114.8875 105.325) (width 0.2) (layer "F.Cu") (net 8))
 (segment (start 138.17 110.33) (end 118.34 110.33) (width 0.2) (layer "F.Cu") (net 10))
 (segment (start 118.15 110.14) (end 118.34 110.33) (width 0.2) (layer "F.Cu") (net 10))
 (segment (start 116.84 110.14) (end 118.15 110.14) (width 0.2) (layer "F.Cu") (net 10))
 (segment (start 153.96 94.54) (end 138.17 110.33) (width 0.2) (layer "F.Cu") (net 10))
 (segment (start 126 104) (end 125.975 104.025) (width 0.2) (layer "F.Cu") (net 5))
 (segment (start 111.84013 106.32) (end 112 106.32) (width 0.2) (layer "F.Cu") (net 11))
 (segment (start 111.499 105.97887) (end 111.84013 106.32) (width 0.2) (layer "F.Cu") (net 11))
 (segment (start 115.66 110) (end 116.16 109.5) (width 0.2) (layer "F.Cu") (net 2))
 (segment (start 116.16 109.5) (end 116.84 109.5) (width 0.2) (layer "F.Cu") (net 2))
 (segment (start 112.5 103.51) (end 113.665 104.675) (width 0.2) (layer "F.Cu") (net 7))
 (segment (start 113.665 104.675) (end 114.8875 104.675) (width 0.2) (layer "F.Cu") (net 7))
 (segment (start 112 105.68) (end 112.18 105.68) (width 0.2) (layer "F.Cu") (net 1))
 (segment (start 112.18 105.68) (end 115.140001 108.64) (width 0.2) (layer "F.Cu") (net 1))
 (segment (start 115.02 108.96) (end 115.34 108.64) (width 0.2) (layer "F.Cu") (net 1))
 (segment (start 115.02 110) (end 115.02 108.96) (width 0.2) (layer "F.Cu") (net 1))
 (segment (start 115.140001 108.64) (end 115.34 108.64) (width 0.2) (layer "F.Cu") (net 1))
 (segment (start 120.49 102.49) (end 120.5 102.5) (width 0.2) (layer "F.Cu") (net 4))
 (segment (start 120.5 107.15) (end 120.5 105.98013) (width 0.2) (layer "F.Cu") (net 4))
 (segment (start 120.5 105.98013) (end 119.84487 105.325) (width 0.2) (layer "F.Cu") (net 4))
 (segment (start 112.5 102.49) (end 120.49 102.49) (width 0.2) (layer "F.Cu") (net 4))
 (segment (start 118.34 109.31) (end 120.5 107.15) (width 0.2) (layer "F.Cu") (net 4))
 (segment (start 118.34 109.31) (end 118.34 109.16) (width 0.2) (layer "F.Cu") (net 4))
 (segment (start 119.84487 105.325) (end 119.1125 105.325) (width 0.2) (layer "F.Cu") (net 4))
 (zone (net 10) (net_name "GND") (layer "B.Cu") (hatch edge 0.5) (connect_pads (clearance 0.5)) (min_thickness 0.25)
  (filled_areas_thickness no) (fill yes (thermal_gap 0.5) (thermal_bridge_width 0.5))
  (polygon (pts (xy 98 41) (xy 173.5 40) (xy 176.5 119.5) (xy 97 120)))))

